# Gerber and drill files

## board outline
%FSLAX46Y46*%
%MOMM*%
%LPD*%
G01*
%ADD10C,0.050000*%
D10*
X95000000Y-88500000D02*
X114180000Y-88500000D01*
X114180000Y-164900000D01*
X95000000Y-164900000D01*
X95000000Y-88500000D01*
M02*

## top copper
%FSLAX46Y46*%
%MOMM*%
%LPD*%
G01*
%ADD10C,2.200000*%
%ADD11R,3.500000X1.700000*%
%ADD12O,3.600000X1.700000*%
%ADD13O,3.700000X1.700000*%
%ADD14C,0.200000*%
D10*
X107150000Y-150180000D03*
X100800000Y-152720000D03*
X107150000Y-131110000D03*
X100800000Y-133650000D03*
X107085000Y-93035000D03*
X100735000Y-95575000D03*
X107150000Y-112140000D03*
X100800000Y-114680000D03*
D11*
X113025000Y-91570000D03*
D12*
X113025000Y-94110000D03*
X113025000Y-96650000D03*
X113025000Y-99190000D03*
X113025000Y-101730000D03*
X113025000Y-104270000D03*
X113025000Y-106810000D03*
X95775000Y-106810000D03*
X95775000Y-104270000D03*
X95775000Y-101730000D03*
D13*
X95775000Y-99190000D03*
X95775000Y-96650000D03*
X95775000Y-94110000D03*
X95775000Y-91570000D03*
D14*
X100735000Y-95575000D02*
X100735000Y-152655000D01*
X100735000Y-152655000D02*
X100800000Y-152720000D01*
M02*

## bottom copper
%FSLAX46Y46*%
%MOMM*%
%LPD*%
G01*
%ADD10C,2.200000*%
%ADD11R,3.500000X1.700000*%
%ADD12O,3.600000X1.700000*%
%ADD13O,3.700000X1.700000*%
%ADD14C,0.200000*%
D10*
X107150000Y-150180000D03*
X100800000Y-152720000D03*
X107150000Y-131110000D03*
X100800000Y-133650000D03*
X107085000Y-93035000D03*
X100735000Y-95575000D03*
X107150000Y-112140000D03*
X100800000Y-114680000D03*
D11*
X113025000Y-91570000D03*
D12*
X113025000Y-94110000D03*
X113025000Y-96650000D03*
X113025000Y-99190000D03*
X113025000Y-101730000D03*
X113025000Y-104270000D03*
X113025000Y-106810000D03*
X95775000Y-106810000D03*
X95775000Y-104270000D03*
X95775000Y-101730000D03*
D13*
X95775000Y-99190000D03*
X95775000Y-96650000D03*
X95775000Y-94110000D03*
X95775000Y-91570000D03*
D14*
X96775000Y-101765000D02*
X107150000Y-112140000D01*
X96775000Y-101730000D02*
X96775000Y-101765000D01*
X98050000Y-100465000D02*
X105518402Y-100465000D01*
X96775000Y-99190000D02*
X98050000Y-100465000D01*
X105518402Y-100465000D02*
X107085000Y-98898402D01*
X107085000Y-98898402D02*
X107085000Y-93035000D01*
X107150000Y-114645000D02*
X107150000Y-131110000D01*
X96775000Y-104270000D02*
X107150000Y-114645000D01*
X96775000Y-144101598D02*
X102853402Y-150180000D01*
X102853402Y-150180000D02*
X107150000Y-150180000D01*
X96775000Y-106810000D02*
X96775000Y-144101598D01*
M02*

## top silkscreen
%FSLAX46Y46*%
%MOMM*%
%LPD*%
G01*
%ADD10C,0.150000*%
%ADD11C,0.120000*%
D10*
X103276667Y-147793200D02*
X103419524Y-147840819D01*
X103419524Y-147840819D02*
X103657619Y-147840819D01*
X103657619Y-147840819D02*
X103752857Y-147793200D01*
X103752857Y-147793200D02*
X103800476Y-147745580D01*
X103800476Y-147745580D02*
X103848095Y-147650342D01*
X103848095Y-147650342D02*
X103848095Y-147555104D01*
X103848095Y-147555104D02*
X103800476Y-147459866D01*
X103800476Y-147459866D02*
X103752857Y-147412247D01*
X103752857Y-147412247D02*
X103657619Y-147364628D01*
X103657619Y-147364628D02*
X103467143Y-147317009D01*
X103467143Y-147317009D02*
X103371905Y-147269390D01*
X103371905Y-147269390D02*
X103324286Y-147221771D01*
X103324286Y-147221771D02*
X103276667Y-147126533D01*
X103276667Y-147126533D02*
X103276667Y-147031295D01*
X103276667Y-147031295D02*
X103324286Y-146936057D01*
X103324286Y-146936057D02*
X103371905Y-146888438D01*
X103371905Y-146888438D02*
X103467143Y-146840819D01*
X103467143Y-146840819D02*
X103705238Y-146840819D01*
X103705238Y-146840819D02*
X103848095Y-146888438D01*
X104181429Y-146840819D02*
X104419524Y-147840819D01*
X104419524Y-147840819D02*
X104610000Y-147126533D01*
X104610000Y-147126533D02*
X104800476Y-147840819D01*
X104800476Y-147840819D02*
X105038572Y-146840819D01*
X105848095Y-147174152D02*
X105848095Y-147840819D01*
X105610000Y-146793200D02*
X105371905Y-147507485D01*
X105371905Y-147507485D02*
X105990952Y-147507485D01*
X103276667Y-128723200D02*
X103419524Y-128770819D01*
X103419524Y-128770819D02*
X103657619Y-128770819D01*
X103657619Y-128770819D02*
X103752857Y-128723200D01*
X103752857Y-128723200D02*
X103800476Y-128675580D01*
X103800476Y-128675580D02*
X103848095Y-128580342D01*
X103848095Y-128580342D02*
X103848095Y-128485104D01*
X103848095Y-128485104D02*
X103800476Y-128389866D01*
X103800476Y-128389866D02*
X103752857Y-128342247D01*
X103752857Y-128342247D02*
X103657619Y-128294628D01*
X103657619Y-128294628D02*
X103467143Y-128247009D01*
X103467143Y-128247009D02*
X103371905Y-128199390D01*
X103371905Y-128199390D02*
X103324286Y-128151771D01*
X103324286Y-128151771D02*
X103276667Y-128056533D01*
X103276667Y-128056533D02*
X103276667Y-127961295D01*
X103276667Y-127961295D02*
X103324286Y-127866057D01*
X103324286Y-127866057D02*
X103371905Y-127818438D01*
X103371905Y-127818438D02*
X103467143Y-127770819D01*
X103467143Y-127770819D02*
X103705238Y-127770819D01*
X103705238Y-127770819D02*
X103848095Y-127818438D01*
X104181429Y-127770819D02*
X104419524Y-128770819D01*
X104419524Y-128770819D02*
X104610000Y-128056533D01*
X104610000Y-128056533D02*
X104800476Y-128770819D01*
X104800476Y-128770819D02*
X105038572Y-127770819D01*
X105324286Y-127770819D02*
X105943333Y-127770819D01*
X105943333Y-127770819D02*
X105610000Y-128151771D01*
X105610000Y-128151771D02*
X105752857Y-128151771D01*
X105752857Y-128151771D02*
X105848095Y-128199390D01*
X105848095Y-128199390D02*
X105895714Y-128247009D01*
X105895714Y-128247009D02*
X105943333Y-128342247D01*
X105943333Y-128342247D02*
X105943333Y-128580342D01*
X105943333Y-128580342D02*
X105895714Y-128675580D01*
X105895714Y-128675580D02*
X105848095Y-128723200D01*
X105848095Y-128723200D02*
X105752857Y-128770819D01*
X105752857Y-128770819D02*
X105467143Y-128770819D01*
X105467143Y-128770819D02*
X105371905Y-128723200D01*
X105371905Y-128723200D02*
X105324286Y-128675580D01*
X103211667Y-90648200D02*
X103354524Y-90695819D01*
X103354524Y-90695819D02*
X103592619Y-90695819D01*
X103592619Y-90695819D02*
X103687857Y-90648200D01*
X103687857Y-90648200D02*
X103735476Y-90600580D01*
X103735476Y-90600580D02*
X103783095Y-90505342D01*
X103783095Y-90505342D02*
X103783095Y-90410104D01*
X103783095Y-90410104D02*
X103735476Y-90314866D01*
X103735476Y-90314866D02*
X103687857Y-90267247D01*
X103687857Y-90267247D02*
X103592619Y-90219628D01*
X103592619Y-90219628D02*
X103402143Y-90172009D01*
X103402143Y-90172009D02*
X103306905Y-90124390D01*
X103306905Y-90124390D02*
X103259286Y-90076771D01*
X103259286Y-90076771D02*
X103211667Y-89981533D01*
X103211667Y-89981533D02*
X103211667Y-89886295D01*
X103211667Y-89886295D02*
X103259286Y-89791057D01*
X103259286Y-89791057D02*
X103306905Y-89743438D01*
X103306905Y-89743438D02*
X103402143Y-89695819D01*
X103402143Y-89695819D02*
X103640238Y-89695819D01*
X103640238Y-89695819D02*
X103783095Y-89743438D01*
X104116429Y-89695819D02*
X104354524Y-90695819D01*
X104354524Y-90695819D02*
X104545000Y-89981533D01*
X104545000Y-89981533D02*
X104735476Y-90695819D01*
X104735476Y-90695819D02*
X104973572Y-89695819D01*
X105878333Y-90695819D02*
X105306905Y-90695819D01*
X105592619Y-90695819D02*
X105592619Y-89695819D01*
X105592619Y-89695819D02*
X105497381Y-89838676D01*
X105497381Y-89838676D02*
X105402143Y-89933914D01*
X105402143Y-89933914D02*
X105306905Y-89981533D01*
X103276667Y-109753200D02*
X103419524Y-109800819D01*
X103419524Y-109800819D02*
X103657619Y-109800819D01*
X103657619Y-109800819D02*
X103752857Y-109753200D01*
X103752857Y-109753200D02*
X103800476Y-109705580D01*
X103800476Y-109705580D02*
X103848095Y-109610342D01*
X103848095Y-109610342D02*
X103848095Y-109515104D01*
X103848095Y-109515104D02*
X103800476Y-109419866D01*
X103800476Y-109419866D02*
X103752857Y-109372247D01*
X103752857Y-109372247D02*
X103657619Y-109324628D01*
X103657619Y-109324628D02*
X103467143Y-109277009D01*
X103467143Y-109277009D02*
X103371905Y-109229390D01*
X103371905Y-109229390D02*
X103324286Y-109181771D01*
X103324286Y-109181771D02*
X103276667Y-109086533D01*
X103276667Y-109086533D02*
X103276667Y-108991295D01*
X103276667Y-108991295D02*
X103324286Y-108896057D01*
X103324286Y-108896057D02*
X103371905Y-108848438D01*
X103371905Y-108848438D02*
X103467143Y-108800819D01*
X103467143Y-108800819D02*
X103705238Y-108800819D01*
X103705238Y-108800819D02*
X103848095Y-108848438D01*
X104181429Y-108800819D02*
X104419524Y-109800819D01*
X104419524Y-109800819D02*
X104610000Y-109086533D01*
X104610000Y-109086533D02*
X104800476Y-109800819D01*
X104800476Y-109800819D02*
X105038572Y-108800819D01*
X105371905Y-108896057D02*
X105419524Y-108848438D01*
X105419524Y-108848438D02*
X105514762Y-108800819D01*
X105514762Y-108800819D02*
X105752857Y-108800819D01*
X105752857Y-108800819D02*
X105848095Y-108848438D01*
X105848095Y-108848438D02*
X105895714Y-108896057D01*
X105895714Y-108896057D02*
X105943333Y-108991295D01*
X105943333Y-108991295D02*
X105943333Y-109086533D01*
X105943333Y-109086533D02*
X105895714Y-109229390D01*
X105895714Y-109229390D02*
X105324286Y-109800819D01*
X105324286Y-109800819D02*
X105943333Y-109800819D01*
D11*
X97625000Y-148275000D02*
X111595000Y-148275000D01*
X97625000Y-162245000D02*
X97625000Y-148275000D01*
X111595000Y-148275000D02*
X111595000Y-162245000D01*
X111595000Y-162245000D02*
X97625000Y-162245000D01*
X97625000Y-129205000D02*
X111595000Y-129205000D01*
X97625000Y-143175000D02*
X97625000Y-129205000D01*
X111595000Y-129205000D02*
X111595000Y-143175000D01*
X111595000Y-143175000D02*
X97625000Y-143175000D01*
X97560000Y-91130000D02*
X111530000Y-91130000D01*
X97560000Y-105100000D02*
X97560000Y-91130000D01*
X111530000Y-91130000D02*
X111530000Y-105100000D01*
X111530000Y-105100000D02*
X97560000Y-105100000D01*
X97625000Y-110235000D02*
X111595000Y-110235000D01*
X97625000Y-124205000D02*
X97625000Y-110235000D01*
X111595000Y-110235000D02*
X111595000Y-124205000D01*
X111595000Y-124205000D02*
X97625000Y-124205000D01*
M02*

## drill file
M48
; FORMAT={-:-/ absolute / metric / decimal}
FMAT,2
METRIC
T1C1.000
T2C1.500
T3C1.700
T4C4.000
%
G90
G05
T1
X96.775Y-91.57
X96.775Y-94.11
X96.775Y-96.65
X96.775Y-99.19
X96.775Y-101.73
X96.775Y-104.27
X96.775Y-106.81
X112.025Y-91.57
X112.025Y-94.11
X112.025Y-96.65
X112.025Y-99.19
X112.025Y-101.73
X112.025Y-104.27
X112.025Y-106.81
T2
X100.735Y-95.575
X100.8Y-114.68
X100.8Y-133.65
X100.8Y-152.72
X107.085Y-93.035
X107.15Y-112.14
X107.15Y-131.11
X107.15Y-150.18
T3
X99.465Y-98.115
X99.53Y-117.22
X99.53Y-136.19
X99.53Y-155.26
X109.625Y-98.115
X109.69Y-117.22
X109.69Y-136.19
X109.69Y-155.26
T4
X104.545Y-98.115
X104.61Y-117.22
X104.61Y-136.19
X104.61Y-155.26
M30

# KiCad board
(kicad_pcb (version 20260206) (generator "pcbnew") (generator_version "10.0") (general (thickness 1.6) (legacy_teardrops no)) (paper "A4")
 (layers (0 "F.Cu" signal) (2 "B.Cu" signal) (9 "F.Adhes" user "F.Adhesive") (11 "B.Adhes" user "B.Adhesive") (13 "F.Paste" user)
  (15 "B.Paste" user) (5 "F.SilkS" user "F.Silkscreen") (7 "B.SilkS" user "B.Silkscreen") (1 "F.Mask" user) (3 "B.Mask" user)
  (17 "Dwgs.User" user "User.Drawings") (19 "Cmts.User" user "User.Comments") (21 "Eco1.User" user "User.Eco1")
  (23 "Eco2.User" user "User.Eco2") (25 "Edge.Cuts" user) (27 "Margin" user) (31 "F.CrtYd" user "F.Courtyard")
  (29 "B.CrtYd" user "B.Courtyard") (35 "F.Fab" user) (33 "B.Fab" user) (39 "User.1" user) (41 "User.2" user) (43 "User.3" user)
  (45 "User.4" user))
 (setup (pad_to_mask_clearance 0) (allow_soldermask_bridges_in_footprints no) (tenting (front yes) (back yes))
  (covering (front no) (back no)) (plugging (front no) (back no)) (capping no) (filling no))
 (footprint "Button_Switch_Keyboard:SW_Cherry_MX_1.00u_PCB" (layer "F.Cu") (at 107.15 150.18)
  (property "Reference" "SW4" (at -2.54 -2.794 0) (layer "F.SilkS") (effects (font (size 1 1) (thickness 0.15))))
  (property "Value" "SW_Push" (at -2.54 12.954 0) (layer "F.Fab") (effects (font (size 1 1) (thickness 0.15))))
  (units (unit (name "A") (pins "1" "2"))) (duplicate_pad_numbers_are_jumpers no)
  (fp_line (start -9.525 -1.905) (end 4.445 -1.905) (stroke (width 0.12) (type solid)) (layer "F.SilkS"))
  (fp_line (start -9.525 12.065) (end -9.525 -1.905) (stroke (width 0.12) (type solid)) (layer "F.SilkS"))
  (fp_line (start 4.445 -1.905) (end 4.445 12.065) (stroke (width 0.12) (type solid)) (layer "F.SilkS"))
  (fp_line (start 4.445 12.065) (end -9.525 12.065) (stroke (width 0.12) (type solid)) (layer "F.SilkS"))
  (pad "" np_thru_hole circle (at -7.62 5.08) (size 1.7 1.7) (drill 1.7) (layers "*.Cu" "*.Mask"))
  (pad "" np_thru_hole circle (at -2.54 5.08) (size 4 4) (drill 4) (layers "*.Cu" "*.Mask"))
  (pad "" np_thru_hole circle (at 2.54 5.08) (size 1.7 1.7) (drill 1.7) (layers "*.Cu" "*.Mask"))
  (pad "1" thru_hole circle (at 0 0) (size 2.2 2.2) (drill 1.5) (layers "*.Cu" "*.Mask") (remove_unused_layers no)
   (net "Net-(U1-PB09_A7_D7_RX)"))
  (pad "2" thru_hole circle (at -6.35 2.54) (size 2.2 2.2) (drill 1.5) (layers "*.Cu" "*.Mask") (remove_unused_layers no) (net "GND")))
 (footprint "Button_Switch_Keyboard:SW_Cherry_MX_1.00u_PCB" (layer "F.Cu") (at 107.15 131.11)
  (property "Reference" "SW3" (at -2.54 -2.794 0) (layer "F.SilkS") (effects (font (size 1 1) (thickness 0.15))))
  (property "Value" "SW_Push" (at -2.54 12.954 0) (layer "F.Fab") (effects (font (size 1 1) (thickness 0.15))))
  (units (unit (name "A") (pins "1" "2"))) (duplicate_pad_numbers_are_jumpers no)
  (fp_line (start -9.525 -1.905) (end 4.445 -1.905) (stroke (width 0.12) (type solid)) (layer "F.SilkS"))
  (fp_line (start -9.525 12.065) (end -9.525 -1.905) (stroke (width 0.12) (type solid)) (layer "F.SilkS"))
  (fp_line (start 4.445 -1.905) (end 4.445 12.065) (stroke (width 0.12) (type solid)) (layer "F.SilkS"))
  (fp_line (start 4.445 12.065) (end -9.525 12.065) (stroke (width 0.12) (type solid)) (layer "F.SilkS"))
  (pad "" np_thru_hole circle (at -7.62 5.08) (size 1.7 1.7) (drill 1.7) (layers "*.Cu" "*.Mask"))
  (pad "" np_thru_hole circle (at -2.54 5.08) (size 4 4) (drill 4) (layers "*.Cu" "*.Mask"))
  (pad "" np_thru_hole circle (at 2.54 5.08) (size 1.7 1.7) (drill 1.7) (layers "*.Cu" "*.Mask"))
  (pad "1" thru_hole circle (at 0 0) (size 2.2 2.2) (drill 1.5) (layers "*.Cu" "*.Mask") (remove_unused_layers no)
   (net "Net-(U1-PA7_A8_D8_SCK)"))
  (pad "2" thru_hole circle (at -6.35 2.54) (size 2.2 2.2) (drill 1.5) (layers "*.Cu" "*.Mask") (remove_unused_layers no) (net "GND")))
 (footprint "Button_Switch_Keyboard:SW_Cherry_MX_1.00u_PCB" (layer "F.Cu") (at 107.085 93.035)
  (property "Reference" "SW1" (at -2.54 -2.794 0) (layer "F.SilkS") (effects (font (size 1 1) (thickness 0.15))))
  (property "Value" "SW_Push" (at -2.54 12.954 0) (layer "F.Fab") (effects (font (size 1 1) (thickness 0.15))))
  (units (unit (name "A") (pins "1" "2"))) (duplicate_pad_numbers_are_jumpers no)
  (fp_line (start -9.525 -1.905) (end 4.445 -1.905) (stroke (width 0.12) (type solid)) (layer "F.SilkS"))
  (fp_line (start -9.525 12.065) (end -9.525 -1.905) (stroke (width 0.12) (type solid)) (layer "F.SilkS"))
  (fp_line (start 4.445 -1.905) (end 4.445 12.065) (stroke (width 0.12) (type solid)) (layer "F.SilkS"))
  (fp_line (start 4.445 12.065) (end -9.525 12.065) (stroke (width 0.12) (type solid)) (layer "F.SilkS"))
  (pad "" np_thru_hole circle (at -7.62 5.08) (size 1.7 1.7) (drill 1.7) (layers "*.Cu" "*.Mask"))
  (pad "" np_thru_hole circle (at -2.54 5.08) (size 4 4) (drill 4) (layers "*.Cu" "*.Mask"))
  (pad "" np_thru_hole circle (at 2.54 5.08) (size 1.7 1.7) (drill 1.7) (layers "*.Cu" "*.Mask"))
  (pad "1" thru_hole circle (at 0 0) (size 2.2 2.2) (drill 1.5) (layers "*.Cu" "*.Mask") (remove_unused_layers no)
   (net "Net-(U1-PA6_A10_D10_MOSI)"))
  (pad "2" thru_hole circle (at -6.35 2.54) (size 2.2 2.2) (drill 1.5) (layers "*.Cu" "*.Mask") (remove_unused_layers no) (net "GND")))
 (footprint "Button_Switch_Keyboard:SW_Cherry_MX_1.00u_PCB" (layer "F.Cu") (at 107.15 112.14)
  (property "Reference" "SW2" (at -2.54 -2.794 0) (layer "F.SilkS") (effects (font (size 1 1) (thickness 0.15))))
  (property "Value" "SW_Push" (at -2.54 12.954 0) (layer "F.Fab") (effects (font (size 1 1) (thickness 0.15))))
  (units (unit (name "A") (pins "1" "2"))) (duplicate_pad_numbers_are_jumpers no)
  (fp_line (start -9.525 -1.905) (end 4.445 -1.905) (stroke (width 0.12) (type solid)) (layer "F.SilkS"))
  (fp_line (start -9.525 12.065) (end -9.525 -1.905) (stroke (width 0.12) (type solid)) (layer "F.SilkS"))
  (fp_line (start 4.445 -1.905) (end 4.445 12.065) (stroke (width 0.12) (type solid)) (layer "F.SilkS"))
  (fp_line (start 4.445 12.065) (end -9.525 12.065) (stroke (width 0.12) (type solid)) (layer "F.SilkS"))
  (pad "" np_thru_hole circle (at -7.62 5.08) (size 1.7 1.7) (drill 1.7) (layers "*.Cu" "*.Mask"))
  (pad "" np_thru_hole circle (at -2.54 5.08) (size 4 4) (drill 4) (layers "*.Cu" "*.Mask"))
  (pad "" np_thru_hole circle (at 2.54 5.08) (size 1.7 1.7) (drill 1.7) (layers "*.Cu" "*.Mask"))
  (pad "1" thru_hole circle (at 0 0) (size 2.2 2.2) (drill 1.5) (layers "*.Cu" "*.Mask") (remove_unused_layers no)
   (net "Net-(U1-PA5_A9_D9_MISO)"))
  (pad "2" thru_hole circle (at -6.35 2.54) (size 2.2 2.2) (drill 1.5) (layers "*.Cu" "*.Mask") (remove_unused_layers no) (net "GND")))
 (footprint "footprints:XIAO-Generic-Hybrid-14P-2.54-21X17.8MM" (layer "B.Cu") (at 104.4 99.19 180)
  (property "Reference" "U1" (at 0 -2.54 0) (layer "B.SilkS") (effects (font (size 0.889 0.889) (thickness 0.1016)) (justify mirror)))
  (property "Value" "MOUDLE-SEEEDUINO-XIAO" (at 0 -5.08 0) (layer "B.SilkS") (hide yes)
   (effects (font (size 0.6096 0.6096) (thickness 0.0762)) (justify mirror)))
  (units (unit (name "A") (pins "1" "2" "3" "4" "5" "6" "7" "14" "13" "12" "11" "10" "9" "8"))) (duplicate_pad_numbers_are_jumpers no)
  (pad "1" thru_hole rect (at -7.625 7.62 180) (size 3.5 1.7) (drill 1 (offset -1 0)) (layers "*.Cu" "*.Mask") (remove_unused_layers no)
   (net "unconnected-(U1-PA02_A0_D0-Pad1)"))
  (pad "2" thru_hole oval (at -7.625 5.08 180) (size 3.6 1.7) (drill 1 (offset -1 0)) (layers "*.Cu" "*.Mask") (remove_unused_layers no)
   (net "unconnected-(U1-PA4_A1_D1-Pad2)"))
  (pad "3" thru_hole oval (at -7.625 2.54 180) (size 3.6 1.7) (drill 1 (offset -1 0)) (layers "*.Cu" "*.Mask") (remove_unused_layers no)
   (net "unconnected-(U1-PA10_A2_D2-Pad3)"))
  (pad "4" thru_hole oval (at -7.625 0 180) (size 3.6 1.7) (drill 1 (offset -1 0)) (layers "*.Cu" "*.Mask") (remove_unused_layers no)
   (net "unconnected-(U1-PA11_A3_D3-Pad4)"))
  (pad "5" thru_hole oval (at -7.625 -2.54 180) (size 3.6 1.7) (drill 1 (offset -1 0)) (layers "*.Cu" "*.Mask") (remove_unused_layers no)
   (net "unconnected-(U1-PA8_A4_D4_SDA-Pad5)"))
  (pad "6" thru_hole oval (at -7.625 -5.08) (size 3.6 1.7) (drill 1 (offset 1 0)) (layers "*.Cu" "*.Mask") (remove_unused_layers no)
   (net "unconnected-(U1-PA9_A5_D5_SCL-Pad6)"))
  (pad "7" thru_hole oval (at -7.625 -7.62 180) (size 3.6 1.7) (drill 1 (offset -1 0)) (layers "*.Cu" "*.Mask") (remove_unused_layers no)
   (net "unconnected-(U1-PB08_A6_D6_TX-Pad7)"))
  (pad "8" thru_hole oval (at 7.625 -7.62 180) (size 3.6 1.7) (drill 1 (offset 1 0)) (layers "*.Cu" "*.Mask") (remove_unused_layers no)
   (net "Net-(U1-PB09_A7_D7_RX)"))
  (pad "9" thru_hole oval (at 7.625 -5.08 180) (size 3.6 1.7) (drill 1 (offset 1 0)) (layers "*.Cu" "*.Mask") (remove_unused_layers no)
   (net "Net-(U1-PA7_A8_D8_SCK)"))
  (pad "10" thru_hole oval (at 7.625 -2.54 180) (size 3.6 1.7) (drill 1 (offset 1 0)) (layers "*.Cu" "*.Mask") (remove_unused_layers no)
   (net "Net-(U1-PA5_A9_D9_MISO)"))
  (pad "11" thru_hole oval (at 7.625 0 180) (size 3.7 1.7) (drill 1 (offset 1 0)) (layers "*.Cu" "*.Mask") (remove_unused_layers no)
   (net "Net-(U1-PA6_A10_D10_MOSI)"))
  (pad "12" thru_hole oval (at 7.625 2.54 180) (size 3.7 1.7) (drill 1 (offset 1 0)) (layers "*.Cu" "*.Mask") (remove_unused_layers no)
   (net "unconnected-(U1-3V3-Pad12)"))
  (pad "13" thru_hole oval (at 7.625 5.08 180) (size 3.7 1.7) (drill 1 (offset 1 0)) (layers "*.Cu" "*.Mask") (remove_unused_layers no)
   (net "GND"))
  (pad "14" thru_hole oval (at 7.625 7.62 180) (size 3.7 1.7) (drill 1 (offset 1 0)) (layers "*.Cu" "*.Mask") (remove_unused_layers no)
   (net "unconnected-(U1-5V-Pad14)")))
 (gr_rect (start 95 88.5) (end 114.18 164.9) (stroke (width 0.05) (type default)) (fill no) (layer "Edge.Cuts"))
 (segment (start 96.775 101.765) (end 107.15 112.14) (width 0.2) (layer "B.Cu") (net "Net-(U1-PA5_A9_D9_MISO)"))
 (segment (start 96.775 101.73) (end 96.775 101.765) (width 0.2) (layer "B.Cu") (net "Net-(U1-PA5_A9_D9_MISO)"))
 (segment (start 100.735 95.575) (end 100.735 152.655) (width 0.2) (layer "F.Cu") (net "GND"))
 (segment (start 100.735 152.655) (end 100.8 152.72) (width 0.2) (layer "F.Cu") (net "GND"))
 (segment (start 98.05 100.465) (end 105.518402 100.465) (width 0.2) (layer "B.Cu") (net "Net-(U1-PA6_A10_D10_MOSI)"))
 (segment (start 96.775 99.19) (end 98.05 100.465) (width 0.2) (layer "B.Cu") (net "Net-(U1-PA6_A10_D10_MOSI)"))
 (segment (start 105.518402 100.465) (end 107.085 98.898402) (width 0.2) (layer "B.Cu") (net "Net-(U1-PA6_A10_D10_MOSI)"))
 (segment (start 107.085 98.898402) (end 107.085 93.035) (width 0.2) (layer "B.Cu") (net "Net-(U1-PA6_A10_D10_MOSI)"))
 (segment (start 107.15 114.645) (end 107.15 131.11) (width 0.2) (layer "B.Cu") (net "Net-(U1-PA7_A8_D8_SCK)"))
 (segment (start 96.775 104.27) (end 107.15 114.645) (width 0.2) (layer "B.Cu") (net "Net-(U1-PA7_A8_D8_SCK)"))
 (segment (start 96.775 144.101598) (end 102.853402 150.18) (width 0.2) (layer "B.Cu") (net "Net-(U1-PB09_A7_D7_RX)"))
 (segment (start 102.853402 150.18) (end 107.15 150.18) (width 0.2) (layer "B.Cu") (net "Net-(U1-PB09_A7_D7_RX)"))
 (segment (start 96.775 106.81) (end 96.775 144.101598) (width 0.2) (layer "B.Cu") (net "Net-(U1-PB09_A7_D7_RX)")))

